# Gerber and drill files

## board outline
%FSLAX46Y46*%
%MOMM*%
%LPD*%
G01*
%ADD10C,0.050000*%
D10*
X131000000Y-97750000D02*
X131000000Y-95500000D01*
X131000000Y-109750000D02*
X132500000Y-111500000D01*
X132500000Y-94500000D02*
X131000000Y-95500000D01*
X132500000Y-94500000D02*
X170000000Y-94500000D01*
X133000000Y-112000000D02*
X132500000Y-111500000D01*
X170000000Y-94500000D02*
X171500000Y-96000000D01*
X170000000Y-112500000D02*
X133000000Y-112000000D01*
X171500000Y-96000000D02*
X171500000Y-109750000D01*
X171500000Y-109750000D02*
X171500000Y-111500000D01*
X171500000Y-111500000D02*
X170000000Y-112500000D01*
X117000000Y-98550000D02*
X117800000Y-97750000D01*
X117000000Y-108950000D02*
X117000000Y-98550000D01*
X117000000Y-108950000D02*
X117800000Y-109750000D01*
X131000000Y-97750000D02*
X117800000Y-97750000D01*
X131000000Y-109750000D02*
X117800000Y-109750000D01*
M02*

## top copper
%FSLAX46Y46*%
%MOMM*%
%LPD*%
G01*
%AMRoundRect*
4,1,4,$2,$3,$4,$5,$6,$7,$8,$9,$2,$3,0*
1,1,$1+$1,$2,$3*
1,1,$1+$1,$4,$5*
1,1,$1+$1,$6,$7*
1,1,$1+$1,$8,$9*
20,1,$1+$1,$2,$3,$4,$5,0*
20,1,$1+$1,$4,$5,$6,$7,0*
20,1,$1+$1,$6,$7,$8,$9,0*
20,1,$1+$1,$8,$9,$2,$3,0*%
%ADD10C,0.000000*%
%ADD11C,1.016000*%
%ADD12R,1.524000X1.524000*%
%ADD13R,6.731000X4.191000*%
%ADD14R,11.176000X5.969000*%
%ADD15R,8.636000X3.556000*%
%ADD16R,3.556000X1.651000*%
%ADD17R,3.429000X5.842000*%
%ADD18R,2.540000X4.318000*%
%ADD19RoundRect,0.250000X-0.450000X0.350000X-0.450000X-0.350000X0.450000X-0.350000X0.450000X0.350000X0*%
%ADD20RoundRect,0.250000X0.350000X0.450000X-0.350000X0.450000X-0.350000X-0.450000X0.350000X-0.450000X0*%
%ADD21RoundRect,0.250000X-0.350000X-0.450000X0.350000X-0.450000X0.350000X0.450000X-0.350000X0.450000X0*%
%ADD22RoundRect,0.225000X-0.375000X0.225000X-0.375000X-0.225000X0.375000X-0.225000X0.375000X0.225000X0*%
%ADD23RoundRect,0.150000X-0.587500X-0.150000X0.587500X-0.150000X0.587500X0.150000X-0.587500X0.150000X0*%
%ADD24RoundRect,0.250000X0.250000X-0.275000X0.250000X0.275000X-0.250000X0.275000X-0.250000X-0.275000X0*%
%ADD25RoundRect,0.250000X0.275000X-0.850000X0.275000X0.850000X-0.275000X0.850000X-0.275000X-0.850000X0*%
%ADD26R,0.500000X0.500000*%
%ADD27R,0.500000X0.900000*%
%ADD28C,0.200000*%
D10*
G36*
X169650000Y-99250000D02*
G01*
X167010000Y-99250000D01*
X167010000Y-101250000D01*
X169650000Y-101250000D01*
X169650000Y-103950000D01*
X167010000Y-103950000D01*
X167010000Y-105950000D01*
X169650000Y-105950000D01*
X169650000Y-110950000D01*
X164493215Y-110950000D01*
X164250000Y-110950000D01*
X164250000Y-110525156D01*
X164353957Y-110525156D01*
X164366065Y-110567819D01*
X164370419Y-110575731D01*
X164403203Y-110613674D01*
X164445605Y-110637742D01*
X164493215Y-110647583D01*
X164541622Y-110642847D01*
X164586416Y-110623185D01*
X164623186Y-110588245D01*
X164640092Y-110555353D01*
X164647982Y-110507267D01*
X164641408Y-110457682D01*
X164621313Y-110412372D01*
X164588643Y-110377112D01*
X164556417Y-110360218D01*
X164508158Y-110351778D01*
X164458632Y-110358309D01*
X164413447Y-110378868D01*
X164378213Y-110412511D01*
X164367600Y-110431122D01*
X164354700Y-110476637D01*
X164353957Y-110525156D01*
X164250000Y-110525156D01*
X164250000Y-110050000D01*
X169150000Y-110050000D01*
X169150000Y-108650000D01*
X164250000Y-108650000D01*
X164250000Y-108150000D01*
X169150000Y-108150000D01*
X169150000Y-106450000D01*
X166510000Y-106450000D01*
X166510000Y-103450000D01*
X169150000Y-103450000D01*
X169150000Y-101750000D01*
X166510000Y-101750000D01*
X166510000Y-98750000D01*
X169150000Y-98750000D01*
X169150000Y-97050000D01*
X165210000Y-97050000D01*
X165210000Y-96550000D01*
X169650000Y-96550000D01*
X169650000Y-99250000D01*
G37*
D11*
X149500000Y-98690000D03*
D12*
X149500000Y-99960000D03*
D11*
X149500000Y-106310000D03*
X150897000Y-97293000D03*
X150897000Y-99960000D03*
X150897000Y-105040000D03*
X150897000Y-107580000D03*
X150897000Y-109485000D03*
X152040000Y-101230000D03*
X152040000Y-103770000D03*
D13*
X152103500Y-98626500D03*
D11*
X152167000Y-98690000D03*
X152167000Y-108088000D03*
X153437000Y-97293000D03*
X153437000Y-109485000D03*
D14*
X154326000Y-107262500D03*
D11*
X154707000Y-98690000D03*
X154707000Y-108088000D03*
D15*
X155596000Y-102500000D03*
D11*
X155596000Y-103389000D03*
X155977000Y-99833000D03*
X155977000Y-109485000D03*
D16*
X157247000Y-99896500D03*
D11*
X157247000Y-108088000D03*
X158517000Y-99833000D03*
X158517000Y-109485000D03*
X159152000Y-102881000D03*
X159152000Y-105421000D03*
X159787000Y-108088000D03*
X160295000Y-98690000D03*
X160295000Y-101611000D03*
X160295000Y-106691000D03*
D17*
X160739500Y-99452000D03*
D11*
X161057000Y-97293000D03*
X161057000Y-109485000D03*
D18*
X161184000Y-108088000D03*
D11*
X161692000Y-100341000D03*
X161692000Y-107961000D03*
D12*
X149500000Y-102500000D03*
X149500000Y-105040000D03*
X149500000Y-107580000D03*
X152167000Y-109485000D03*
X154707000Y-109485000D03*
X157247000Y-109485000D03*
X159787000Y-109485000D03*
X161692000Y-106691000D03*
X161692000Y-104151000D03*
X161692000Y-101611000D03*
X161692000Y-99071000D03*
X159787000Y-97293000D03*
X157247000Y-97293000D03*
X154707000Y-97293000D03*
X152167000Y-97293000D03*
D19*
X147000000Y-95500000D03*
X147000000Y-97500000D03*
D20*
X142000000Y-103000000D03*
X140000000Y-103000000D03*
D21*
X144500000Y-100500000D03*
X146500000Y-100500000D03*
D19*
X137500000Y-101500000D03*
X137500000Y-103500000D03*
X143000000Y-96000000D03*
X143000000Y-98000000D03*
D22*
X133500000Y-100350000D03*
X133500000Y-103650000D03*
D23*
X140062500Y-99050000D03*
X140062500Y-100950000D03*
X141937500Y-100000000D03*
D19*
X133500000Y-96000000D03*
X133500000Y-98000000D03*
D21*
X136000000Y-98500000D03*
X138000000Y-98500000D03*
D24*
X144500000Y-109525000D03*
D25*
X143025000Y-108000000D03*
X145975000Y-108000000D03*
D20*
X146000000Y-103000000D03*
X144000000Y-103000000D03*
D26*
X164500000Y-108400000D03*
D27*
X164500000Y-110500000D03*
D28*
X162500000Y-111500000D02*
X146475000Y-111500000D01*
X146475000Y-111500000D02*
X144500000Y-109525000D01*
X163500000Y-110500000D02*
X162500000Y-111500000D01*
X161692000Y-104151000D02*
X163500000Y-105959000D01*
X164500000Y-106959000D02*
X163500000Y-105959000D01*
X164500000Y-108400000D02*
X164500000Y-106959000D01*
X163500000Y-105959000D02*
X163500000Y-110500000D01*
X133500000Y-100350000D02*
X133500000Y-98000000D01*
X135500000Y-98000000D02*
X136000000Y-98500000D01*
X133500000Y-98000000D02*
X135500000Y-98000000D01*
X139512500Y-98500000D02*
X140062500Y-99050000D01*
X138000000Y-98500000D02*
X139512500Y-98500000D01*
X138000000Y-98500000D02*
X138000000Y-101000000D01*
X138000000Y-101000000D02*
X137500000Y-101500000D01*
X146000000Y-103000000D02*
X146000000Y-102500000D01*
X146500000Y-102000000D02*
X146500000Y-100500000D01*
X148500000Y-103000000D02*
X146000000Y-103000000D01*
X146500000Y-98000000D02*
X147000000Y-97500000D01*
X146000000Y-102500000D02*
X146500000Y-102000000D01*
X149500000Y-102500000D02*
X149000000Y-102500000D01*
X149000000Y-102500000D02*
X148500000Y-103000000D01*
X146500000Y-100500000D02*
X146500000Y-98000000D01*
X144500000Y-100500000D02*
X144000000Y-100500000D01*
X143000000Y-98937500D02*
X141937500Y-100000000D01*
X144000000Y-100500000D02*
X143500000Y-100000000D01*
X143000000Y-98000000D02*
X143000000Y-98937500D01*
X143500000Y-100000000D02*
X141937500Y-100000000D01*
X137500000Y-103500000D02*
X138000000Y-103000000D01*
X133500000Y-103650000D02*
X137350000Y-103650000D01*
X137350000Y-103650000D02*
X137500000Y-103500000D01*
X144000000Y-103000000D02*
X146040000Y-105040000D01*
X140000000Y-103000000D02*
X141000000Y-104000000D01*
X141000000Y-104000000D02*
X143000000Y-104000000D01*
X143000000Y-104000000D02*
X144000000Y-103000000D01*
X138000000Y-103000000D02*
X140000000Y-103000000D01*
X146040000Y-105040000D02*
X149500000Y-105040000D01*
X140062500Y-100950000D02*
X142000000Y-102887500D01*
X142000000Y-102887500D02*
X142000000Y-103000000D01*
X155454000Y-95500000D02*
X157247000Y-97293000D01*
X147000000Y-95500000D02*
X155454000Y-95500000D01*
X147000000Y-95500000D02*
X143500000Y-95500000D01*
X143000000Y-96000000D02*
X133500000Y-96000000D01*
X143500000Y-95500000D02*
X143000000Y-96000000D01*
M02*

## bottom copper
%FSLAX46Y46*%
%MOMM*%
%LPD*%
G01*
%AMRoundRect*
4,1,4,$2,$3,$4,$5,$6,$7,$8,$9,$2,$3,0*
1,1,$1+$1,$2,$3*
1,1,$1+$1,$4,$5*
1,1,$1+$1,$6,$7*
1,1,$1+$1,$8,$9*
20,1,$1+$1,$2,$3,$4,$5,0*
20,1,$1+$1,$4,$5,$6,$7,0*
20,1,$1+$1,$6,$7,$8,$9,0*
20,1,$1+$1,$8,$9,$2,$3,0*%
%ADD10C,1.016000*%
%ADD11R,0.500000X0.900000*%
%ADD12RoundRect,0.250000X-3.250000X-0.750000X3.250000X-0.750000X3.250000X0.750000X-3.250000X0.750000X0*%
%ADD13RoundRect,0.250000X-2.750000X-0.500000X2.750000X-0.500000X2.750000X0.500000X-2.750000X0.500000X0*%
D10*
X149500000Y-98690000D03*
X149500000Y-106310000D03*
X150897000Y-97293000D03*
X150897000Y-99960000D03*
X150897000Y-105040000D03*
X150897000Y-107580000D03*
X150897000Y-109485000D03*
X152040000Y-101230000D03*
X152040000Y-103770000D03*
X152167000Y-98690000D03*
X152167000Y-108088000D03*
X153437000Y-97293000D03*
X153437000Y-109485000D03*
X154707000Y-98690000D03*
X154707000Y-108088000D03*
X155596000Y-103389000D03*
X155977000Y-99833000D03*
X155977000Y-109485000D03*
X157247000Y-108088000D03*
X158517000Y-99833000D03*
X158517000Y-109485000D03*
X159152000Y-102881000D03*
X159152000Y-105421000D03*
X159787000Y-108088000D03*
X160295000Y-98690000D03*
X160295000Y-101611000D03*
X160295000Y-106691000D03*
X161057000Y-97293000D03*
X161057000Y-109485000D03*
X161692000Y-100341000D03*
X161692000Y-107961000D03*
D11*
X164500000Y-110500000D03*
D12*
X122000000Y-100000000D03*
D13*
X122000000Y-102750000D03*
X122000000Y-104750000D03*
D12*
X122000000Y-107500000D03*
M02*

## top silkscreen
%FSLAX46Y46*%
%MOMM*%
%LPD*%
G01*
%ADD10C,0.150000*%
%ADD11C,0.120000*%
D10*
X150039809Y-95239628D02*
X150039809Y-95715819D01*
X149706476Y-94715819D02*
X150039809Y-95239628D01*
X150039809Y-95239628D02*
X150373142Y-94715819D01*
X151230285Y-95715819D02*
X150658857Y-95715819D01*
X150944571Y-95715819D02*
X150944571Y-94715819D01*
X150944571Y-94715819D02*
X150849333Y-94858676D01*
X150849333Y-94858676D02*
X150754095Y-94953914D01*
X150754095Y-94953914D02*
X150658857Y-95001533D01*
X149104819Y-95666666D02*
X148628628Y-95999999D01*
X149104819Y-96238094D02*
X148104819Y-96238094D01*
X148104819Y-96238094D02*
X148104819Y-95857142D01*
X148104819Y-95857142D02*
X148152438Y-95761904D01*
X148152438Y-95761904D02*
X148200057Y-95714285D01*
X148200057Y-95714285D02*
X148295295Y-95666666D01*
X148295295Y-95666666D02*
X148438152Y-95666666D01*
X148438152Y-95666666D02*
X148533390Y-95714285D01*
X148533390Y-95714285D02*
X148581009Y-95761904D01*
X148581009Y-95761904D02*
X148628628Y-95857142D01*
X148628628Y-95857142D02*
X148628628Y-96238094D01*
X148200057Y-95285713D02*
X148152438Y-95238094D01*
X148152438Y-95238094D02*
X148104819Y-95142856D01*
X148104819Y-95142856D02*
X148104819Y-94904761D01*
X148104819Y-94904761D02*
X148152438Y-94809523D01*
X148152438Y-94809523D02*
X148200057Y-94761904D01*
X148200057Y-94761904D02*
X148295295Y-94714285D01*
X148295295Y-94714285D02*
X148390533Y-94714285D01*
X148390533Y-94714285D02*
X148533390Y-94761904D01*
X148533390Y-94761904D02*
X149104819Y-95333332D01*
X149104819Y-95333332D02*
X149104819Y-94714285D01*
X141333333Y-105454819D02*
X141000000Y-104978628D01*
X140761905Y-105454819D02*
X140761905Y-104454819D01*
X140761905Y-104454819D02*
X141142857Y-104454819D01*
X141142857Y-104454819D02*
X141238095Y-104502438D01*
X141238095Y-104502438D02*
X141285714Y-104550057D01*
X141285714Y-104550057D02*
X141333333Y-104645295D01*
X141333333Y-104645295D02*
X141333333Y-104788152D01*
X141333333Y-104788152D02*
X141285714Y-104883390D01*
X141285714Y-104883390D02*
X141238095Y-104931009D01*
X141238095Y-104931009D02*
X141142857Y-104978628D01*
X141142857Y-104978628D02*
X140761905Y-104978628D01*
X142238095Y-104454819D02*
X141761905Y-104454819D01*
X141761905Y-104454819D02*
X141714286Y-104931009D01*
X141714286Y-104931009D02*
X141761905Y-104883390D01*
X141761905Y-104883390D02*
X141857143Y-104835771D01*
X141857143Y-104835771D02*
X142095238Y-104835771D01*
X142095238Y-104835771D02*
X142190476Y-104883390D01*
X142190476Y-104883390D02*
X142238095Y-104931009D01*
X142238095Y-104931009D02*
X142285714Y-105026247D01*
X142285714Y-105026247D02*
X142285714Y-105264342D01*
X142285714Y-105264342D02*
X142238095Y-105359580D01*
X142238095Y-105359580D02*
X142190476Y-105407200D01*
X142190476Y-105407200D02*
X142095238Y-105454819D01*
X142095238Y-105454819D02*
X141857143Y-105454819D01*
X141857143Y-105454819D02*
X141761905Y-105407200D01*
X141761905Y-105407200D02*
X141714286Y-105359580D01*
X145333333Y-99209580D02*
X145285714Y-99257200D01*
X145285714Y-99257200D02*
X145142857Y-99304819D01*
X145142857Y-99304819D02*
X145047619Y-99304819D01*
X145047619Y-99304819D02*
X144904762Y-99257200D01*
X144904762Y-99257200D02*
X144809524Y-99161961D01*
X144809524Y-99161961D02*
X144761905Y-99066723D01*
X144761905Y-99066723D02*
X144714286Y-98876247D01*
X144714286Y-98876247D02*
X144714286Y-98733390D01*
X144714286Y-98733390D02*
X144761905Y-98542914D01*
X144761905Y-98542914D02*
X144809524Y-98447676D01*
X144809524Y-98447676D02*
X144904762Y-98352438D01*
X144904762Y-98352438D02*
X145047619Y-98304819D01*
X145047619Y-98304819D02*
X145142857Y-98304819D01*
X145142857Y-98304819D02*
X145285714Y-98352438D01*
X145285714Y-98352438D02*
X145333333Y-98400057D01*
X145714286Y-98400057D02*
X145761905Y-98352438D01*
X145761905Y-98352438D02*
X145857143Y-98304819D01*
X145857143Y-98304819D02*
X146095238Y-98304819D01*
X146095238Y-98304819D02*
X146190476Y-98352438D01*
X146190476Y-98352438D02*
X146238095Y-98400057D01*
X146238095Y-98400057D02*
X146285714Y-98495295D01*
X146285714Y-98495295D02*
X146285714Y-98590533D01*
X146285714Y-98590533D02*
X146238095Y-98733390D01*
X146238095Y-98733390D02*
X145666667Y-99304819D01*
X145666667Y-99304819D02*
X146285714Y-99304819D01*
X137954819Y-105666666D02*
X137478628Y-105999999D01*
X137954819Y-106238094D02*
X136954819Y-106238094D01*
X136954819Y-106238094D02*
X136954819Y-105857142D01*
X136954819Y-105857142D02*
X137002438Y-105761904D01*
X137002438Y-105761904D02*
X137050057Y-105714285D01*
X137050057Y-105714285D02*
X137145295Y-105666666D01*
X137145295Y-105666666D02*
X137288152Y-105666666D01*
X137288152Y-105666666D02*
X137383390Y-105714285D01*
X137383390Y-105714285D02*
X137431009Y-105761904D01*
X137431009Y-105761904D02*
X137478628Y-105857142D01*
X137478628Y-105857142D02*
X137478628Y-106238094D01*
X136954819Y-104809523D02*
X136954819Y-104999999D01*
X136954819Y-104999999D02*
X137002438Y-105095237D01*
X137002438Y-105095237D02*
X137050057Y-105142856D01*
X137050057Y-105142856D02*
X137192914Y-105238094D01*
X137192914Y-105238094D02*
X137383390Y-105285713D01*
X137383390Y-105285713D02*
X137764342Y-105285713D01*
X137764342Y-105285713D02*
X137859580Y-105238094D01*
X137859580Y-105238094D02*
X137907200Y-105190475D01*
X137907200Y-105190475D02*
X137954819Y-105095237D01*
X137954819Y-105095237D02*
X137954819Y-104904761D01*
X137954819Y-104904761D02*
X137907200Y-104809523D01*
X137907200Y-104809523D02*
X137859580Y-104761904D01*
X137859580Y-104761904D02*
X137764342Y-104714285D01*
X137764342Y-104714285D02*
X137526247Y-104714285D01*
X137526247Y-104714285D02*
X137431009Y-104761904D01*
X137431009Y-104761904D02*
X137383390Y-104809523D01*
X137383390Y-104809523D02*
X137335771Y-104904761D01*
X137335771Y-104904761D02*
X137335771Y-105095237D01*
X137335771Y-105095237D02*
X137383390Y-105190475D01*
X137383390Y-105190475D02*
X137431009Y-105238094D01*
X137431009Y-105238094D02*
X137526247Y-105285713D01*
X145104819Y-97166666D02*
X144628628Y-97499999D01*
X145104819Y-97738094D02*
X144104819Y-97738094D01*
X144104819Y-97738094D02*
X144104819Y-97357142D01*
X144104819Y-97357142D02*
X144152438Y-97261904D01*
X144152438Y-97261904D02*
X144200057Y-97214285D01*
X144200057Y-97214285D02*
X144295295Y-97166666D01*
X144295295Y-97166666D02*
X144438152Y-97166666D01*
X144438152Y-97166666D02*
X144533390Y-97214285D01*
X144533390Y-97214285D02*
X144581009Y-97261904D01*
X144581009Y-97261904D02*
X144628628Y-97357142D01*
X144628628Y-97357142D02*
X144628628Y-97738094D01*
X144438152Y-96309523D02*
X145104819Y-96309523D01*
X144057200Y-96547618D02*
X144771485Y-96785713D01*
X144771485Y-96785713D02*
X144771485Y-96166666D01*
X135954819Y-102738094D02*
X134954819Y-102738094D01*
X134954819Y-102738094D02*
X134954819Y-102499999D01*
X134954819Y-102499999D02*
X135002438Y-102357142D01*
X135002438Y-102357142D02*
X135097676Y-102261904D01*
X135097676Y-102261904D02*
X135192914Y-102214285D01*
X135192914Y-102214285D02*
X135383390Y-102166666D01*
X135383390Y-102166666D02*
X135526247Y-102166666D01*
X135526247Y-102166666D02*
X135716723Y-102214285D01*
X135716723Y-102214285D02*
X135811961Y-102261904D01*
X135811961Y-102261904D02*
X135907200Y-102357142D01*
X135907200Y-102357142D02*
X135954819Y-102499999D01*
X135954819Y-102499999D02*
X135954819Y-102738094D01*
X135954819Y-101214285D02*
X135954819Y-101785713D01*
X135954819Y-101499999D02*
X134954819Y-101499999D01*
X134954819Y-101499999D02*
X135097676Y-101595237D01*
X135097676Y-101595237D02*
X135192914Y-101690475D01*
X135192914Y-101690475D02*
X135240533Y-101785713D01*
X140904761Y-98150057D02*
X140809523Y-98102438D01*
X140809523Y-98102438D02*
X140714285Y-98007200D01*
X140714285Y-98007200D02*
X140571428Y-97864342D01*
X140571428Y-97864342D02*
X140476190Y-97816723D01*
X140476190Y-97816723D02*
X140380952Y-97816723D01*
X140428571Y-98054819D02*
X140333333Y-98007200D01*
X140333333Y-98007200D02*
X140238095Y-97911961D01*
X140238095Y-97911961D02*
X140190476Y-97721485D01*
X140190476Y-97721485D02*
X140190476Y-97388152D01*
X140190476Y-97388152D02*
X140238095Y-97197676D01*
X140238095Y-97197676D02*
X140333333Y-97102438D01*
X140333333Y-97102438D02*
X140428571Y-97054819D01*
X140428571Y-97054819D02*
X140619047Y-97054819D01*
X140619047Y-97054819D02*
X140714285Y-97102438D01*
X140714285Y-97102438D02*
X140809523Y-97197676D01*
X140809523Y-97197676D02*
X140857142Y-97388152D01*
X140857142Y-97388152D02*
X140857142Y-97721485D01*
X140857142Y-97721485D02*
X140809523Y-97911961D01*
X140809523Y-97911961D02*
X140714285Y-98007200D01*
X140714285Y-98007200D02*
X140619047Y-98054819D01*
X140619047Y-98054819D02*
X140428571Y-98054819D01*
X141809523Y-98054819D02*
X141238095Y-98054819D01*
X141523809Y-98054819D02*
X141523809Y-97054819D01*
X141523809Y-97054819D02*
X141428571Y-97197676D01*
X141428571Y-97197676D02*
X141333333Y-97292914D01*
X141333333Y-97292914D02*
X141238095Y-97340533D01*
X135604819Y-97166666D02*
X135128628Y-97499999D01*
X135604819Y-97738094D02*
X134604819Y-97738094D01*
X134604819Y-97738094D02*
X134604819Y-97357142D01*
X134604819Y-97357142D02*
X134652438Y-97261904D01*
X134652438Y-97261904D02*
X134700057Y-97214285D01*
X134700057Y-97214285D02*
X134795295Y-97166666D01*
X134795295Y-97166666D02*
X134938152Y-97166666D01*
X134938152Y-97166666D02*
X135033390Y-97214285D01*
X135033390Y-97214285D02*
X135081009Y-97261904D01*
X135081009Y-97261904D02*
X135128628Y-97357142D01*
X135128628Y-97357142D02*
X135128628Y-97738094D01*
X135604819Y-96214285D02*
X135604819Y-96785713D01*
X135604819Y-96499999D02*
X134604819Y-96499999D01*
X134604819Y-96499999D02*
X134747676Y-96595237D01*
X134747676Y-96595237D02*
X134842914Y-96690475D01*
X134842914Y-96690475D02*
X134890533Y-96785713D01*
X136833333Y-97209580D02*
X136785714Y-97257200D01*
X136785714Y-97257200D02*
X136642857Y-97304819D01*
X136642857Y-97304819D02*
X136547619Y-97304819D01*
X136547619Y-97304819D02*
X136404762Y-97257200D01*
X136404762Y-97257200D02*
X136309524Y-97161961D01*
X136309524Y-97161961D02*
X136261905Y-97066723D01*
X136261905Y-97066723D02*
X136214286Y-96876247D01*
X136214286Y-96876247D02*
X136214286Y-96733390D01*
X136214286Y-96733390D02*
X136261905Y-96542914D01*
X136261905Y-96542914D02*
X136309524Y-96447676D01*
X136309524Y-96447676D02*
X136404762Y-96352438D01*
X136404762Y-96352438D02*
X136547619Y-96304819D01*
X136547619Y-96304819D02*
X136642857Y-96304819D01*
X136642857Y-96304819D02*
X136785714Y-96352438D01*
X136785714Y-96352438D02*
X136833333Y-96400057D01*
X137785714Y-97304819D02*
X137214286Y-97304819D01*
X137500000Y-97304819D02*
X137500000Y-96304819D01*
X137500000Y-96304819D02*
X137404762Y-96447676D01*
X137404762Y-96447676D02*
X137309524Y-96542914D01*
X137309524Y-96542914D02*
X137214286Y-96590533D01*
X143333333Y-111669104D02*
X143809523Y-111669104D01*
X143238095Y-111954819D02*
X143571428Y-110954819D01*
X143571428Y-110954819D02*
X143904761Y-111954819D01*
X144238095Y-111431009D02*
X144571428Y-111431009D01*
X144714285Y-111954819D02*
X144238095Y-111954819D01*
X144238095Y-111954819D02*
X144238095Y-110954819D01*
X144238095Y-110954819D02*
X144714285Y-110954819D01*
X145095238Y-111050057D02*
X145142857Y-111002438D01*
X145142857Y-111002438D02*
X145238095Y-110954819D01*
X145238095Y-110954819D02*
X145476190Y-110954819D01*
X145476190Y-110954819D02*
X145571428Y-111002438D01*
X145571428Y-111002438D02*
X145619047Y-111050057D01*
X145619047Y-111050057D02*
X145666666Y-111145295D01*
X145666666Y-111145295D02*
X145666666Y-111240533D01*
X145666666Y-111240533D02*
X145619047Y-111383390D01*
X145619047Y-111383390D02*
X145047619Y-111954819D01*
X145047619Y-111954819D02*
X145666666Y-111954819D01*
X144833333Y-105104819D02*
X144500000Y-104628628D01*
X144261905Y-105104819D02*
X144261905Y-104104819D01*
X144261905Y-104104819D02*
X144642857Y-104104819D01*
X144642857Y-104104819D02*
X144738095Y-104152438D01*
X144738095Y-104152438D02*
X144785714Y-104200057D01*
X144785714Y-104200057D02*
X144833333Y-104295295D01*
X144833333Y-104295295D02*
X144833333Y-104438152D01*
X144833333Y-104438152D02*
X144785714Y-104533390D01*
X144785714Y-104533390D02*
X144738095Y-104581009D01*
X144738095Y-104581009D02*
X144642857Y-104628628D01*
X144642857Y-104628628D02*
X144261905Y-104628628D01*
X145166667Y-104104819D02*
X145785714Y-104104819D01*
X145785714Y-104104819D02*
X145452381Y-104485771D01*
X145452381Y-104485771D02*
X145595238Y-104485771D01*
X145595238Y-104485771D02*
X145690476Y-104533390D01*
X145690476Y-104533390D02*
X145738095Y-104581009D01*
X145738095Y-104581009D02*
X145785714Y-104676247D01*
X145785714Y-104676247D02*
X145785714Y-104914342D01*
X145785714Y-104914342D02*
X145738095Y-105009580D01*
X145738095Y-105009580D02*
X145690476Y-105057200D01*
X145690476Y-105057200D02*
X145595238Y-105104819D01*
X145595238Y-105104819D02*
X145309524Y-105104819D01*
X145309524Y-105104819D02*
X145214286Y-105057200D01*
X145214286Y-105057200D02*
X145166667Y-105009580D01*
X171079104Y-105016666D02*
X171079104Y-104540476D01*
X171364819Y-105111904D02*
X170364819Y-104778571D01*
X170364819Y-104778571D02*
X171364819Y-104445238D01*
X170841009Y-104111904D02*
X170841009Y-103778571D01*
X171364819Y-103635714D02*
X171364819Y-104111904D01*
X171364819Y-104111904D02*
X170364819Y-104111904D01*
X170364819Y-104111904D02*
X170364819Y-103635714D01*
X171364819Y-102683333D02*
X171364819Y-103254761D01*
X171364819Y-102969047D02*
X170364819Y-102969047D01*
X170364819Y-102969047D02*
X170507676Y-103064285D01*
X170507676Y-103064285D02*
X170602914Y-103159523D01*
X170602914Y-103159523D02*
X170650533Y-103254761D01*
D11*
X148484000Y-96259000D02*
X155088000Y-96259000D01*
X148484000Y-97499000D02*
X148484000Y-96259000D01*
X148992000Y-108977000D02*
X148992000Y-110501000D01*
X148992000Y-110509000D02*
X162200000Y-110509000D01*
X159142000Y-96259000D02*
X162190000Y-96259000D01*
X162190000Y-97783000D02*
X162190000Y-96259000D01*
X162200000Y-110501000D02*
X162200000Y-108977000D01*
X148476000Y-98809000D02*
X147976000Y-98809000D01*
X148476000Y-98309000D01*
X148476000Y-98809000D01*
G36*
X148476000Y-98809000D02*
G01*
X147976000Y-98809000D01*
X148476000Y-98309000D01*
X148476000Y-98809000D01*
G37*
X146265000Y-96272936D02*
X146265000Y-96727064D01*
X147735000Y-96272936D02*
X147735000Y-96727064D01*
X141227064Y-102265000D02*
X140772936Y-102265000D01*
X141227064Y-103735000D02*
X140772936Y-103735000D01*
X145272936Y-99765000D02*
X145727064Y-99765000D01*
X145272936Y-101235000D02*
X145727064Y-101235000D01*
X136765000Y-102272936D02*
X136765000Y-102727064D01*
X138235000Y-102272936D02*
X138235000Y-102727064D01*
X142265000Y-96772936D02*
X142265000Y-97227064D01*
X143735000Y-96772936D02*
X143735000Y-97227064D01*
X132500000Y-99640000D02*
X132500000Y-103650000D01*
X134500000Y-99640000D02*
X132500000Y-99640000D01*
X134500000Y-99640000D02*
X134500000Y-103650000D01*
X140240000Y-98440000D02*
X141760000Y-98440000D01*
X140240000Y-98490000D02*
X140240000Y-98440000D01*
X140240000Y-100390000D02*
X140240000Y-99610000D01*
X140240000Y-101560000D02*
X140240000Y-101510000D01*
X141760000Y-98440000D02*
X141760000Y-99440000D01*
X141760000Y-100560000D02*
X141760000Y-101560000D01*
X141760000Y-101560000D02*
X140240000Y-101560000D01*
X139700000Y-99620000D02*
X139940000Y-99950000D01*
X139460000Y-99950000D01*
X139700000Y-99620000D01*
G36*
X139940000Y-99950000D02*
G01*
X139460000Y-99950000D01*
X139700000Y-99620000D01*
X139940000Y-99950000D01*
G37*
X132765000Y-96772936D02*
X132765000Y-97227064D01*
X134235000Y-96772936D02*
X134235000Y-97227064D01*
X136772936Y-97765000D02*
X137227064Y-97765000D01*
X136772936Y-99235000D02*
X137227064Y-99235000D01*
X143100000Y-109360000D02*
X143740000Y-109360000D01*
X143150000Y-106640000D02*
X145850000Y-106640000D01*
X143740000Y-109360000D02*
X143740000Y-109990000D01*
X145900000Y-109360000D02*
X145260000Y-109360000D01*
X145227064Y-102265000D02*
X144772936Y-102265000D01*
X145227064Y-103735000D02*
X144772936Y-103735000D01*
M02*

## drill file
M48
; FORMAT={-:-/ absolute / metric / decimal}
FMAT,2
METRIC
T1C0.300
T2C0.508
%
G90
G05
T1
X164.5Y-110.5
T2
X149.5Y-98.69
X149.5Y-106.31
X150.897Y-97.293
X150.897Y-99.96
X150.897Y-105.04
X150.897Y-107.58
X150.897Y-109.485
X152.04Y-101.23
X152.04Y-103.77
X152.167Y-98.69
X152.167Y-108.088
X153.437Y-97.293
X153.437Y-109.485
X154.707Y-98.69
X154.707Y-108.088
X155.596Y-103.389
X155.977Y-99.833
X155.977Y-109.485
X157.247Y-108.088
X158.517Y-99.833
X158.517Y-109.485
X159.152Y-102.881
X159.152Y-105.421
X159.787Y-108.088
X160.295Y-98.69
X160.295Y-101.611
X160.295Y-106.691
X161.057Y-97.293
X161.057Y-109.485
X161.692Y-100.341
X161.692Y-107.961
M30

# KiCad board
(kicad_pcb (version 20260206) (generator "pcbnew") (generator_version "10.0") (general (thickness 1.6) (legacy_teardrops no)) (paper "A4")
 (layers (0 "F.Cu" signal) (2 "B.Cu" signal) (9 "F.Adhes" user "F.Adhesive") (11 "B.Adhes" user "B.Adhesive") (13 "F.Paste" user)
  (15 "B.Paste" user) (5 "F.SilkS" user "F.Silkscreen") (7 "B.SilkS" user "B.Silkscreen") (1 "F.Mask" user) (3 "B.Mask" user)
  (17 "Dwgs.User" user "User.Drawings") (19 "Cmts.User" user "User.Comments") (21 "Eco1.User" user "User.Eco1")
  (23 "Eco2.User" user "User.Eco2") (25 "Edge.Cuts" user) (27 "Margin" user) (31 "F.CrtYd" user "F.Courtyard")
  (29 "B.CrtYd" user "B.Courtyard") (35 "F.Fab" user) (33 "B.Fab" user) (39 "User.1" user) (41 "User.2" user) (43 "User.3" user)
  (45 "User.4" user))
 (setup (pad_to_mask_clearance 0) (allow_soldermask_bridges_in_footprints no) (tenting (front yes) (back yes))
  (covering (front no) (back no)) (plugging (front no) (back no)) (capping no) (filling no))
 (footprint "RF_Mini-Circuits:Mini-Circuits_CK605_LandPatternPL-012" (layer "F.Cu") (at 155.596 103.389)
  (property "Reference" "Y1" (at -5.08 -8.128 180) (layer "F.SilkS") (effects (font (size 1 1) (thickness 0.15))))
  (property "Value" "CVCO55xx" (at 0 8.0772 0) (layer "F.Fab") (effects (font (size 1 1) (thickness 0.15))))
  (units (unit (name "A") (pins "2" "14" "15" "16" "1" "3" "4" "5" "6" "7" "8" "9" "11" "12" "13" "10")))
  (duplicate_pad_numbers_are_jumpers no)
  (fp_line (start -7.112 -7.13) (end -0.508 -7.13) (stroke (width 0.12) (type solid)) (layer "F.SilkS"))
  (fp_line (start -7.112 -5.89) (end -7.112 -7.13) (stroke (width 0.12) (type solid)) (layer "F.SilkS"))
  (fp_line (start -6.604 5.588) (end -6.604 7.112) (stroke (width 0.12) (type solid)) (layer "F.SilkS"))
  (fp_line (start -6.604 7.12) (end 6.604 7.12) (stroke (width 0.12) (type solid)) (layer "F.SilkS"))
  (fp_line (start 3.546 -7.13) (end 6.594 -7.13) (stroke (width 0.12) (type solid)) (layer "F.SilkS"))
  (fp_line (start 6.594 -5.606) (end 6.594 -7.13) (stroke (width 0.12) (type solid)) (layer "F.SilkS"))
  (fp_line (start 6.604 7.112) (end 6.604 5.588) (stroke (width 0.12) (type solid)) (layer "F.SilkS"))
  (fp_poly
   (pts (xy -7.12 -4.58) (xy -7.62 -4.58) (xy -7.12 -5.08) (xy -7.12 -4.58)) (stroke (width 0.12) (type solid)) (fill yes) (layer "F.SilkS"))
  (pad "1" thru_hole circle (at -6.096 -4.699) (size 1.016 1.016) (drill 0.508) (layers "*.Cu") (remove_unused_layers no) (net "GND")
   (zone_connect 2))
  (pad "1" smd rect (at -6.096 -3.429 270) (size 1.524 1.524) (layers "F.Cu" "F.Mask" "F.Paste") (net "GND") (zone_connect 2))
  (pad "1" thru_hole circle (at -6.096 2.921) (size 1.016 1.016) (drill 0.508) (layers "*.Cu") (remove_unused_layers no) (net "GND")
   (zone_connect 2))
  (pad "1" thru_hole circle (at -4.699 -6.096) (size 1.016 1.016) (drill 0.508) (layers "*.Cu") (remove_unused_layers no) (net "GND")
   (zone_connect 2))
  (pad "1" thru_hole circle (at -4.699 -3.429) (size 1.016 1.016) (drill 0.508) (layers "*.Cu") (remove_unused_layers no) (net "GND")
   (zone_connect 2))
  (pad "1" thru_hole circle (at -4.699 1.651) (size 1.016 1.016) (drill 0.508) (layers "*.Cu") (remove_unused_layers no) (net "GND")
   (zone_connect 2))
  (pad "1" thru_hole circle (at -4.699 4.191) (size 1.016 1.016) (drill 0.508) (layers "*.Cu") (remove_unused_layers no) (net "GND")
   (zone_connect 2))
  (pad "1" thru_hole circle (at -4.699 6.096) (size 1.016 1.016) (drill 0.508) (layers "*.Cu") (remove_unused_layers no) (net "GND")
   (zone_connect 2))
  (pad "1" thru_hole circle (at -3.556 -2.159) (size 1.016 1.016) (drill 0.508) (layers "*.Cu") (remove_unused_layers no) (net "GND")
   (zone_connect 2))
  (pad "1" thru_hole circle (at -3.556 0.381) (size 1.016 1.016) (drill 0.508) (layers "*.Cu") (remove_unused_layers no) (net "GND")
   (zone_connect 2))
  (pad "1" smd rect (at -3.4925 -4.7625) (size 6.731 4.191) (layers "F.Cu") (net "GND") (zone_connect 2))
  (pad "1" thru_hole circle (at -3.429 -4.699) (size 1.016 1.016) (drill 0.508) (layers "*.Cu") (remove_unused_layers no) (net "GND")
   (zone_connect 2))
  (pad "1" thru_hole circle (at -3.429 4.699) (size 1.016 1.016) (drill 0.508) (layers "*.Cu") (remove_unused_layers no) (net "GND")
   (zone_connect 2))
  (pad "1" thru_hole circle (at -2.159 -6.096) (size 1.016 1.016) (drill 0.508) (layers "*.Cu") (remove_unused_layers no) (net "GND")
   (zone_connect 2))
  (pad "1" thru_hole circle (at -2.159 6.096) (size 1.016 1.016) (drill 0.508) (layers "*.Cu") (remove_unused_layers no) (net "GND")
   (zone_connect 2))
  (pad "1" smd rect (at -1.27 3.8735) (size 11.176 5.969) (layers "F.Cu") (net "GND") (zone_connect 2))
  (pad "1" thru_hole circle (at -0.889 -4.699) (size 1.016 1.016) (drill 0.508) (layers "*.Cu") (remove_unused_layers no) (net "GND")
   (zone_connect 2))
  (pad "1" thru_hole circle (at -0.889 4.699) (size 1.016 1.016) (drill 0.508) (layers "*.Cu") (remove_unused_layers no) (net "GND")
   (zone_connect 2))
  (pad "1" smd rect (at 0 -0.889) (size 8.636 3.556) (layers "F.Cu") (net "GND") (zone_connect 2))
  (pad "1" thru_hole circle (at 0 0) (size 1.016 1.016) (drill 0.508) (layers "*.Cu") (remove_unused_layers no) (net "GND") (zone_connect 2))
  (pad "1" thru_hole circle (at 0.381 -3.556) (size 1.016 1.016) (drill 0.508) (layers "*.Cu") (remove_unused_layers no) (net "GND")
   (zone_connect 2))
  (pad "1" thru_hole circle (at 0.381 6.096) (size 1.016 1.016) (drill 0.508) (layers "*.Cu") (remove_unused_layers no) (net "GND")
   (zone_connect 2))
  (pad "1" smd rect (at 1.651 -3.4925) (size 3.556 1.651) (layers "F.Cu") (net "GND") (zone_connect 2))
  (pad "1" thru_hole circle (at 1.651 4.699) (size 1.016 1.016) (drill 0.508) (layers "*.Cu") (remove_unused_layers no) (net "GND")
   (zone_connect 2))
  (pad "1" thru_hole circle (at 2.921 -3.556) (size 1.016 1.016) (drill 0.508) (layers "*.Cu") (remove_unused_layers no) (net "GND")
   (zone_connect 2))
  (pad "1" thru_hole circle (at 2.921 6.096) (size 1.016 1.016) (drill 0.508) (layers "*.Cu") (remove_unused_layers no) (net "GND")
   (zone_connect 2))
  (pad "1" thru_hole circle (at 3.556 -0.508) (size 1.016 1.016) (drill 0.508) (layers "*.Cu") (remove_unused_layers no) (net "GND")
   (zone_connect 2))
  (pad "1" thru_hole circle (at 3.556 2.032) (size 1.016 1.016) (drill 0.508) (layers "*.Cu") (remove_unused_layers no) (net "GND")
   (zone_connect 2))
  (pad "1" thru_hole circle (at 4.191 4.699) (size 1.016 1.016) (drill 0.508) (layers "*.Cu") (remove_unused_layers no) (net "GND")
   (zone_connect 2))
  (pad "1" thru_hole circle (at 4.699 -4.699) (size 1.016 1.016) (drill 0.508) (layers "*.Cu") (remove_unused_layers no) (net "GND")
   (zone_connect 2))
  (pad "1" thru_hole circle (at 4.699 -1.778) (size 1.016 1.016) (drill 0.508) (layers "*.Cu") (remove_unused_layers no) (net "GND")
   (zone_connect 2))
  (pad "1" thru_hole circle (at 4.699 3.302) (size 1.016 1.016) (drill 0.508) (layers "*.Cu") (remove_unused_layers no) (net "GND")
   (zone_connect 2))
  (pad "1" smd rect (at 5.1435 -3.937) (size 3.429 5.842) (layers "F.Cu") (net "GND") (zone_connect 2))
  (pad "1" thru_hole circle (at 5.461 -6.096) (size 1.016 1.016) (drill 0.508) (layers "*.Cu") (remove_unused_layers no) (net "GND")
   (zone_connect 2))
  (pad "1" thru_hole circle (at 5.461 6.096) (size 1.016 1.016) (drill 0.508) (layers "*.Cu") (remove_unused_layers no) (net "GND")
   (zone_connect 2))
  (pad "1" smd rect (at 5.588 4.699) (size 2.54 4.318) (layers "F.Cu") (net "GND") (zone_connect 2))
  (pad "1" thru_hole circle (at 6.096 -3.048) (size 1.016 1.016) (drill 0.508) (layers "*.Cu") (remove_unused_layers no) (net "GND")
   (zone_connect 2))
  (pad "1" thru_hole circle (at 6.096 4.572) (size 1.016 1.016) (drill 0.508) (layers "*.Cu") (remove_unused_layers no) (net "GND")
   (zone_connect 2))
  (pad "2" smd rect (at -6.096 -0.889 270) (size 1.524 1.524) (layers "F.Cu" "F.Mask" "F.Paste") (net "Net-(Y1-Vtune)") (clearance 1.016))
  (pad "3" smd rect (at -6.096 1.651 270) (size 1.524 1.524) (layers "F.Cu" "F.Mask" "F.Paste") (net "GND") (zone_connect 2))
  (pad "4" smd rect (at -6.096 4.191 270) (size 1.524 1.524) (layers "F.Cu" "F.Mask" "F.Paste") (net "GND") (zone_connect 2))
  (pad "5" smd rect (at -3.429 6.096 270) (size 1.524 1.524) (layers "F.Cu" "F.Mask" "F.Paste") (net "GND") (zone_connect 2))
  (pad "6" smd rect (at -0.889 6.096 270) (size 1.524 1.524) (layers "F.Cu" "F.Mask" "F.Paste") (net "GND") (zone_connect 2))
  (pad "7" smd rect (at 1.651 6.096 270) (size 1.524 1.524) (layers "F.Cu" "F.Mask" "F.Paste") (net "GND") (zone_connect 2))
  (pad "8" smd rect (at 4.191 6.096 270) (size 1.524 1.524) (layers "F.Cu" "F.Mask" "F.Paste") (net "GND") (zone_connect 2))
  (pad "9" smd rect (at 6.096 3.302 270) (size 1.524 1.524) (layers "F.Cu" "F.Mask" "F.Paste") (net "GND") (zone_connect 2))
  (pad "10" smd rect (at 6.096 0.762 270) (size 1.524 1.524) (layers "F.Cu" "F.Mask" "F.Paste") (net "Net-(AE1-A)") (clearance 1.016))
  (pad "11" smd rect (at 6.096 -1.778 270) (size 1.524 1.524) (layers "F.Cu" "F.Mask" "F.Paste") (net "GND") (zone_connect 2))
  (pad "12" smd rect (at 6.096 -4.318 270) (size 1.524 1.524) (layers "F.Cu" "F.Mask" "F.Paste") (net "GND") (zone_connect 2))
  (pad "13" smd rect (at 4.191 -6.096 270) (size 1.524 1.524) (layers "F.Cu" "F.Mask" "F.Paste") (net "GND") (zone_connect 2))
  (pad "14" smd rect (at 1.651 -6.096 270) (size 1.524 1.524) (layers "F.Cu" "F.Mask" "F.Paste") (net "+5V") (clearance 1.016))
  (pad "15" smd rect (at -0.889 -6.096 270) (size 1.524 1.524) (layers "F.Cu" "F.Mask" "F.Paste") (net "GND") (zone_connect 2))
  (pad "16" smd rect (at -3.429 -6.096 270) (size 1.524 1.524) (layers "F.Cu" "F.Mask" "F.Paste") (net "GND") (zone_connect 2)))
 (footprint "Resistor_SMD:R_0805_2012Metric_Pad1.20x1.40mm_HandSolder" (layer "F.Cu") (at 147 96.5 -90)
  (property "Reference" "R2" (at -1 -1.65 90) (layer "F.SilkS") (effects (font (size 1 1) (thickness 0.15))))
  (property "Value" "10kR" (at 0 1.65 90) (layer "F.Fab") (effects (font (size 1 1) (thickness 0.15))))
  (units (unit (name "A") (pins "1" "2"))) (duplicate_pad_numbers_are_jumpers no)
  (fp_line (start -0.227064 0.735) (end 0.227064 0.735) (stroke (width 0.12) (type solid)) (layer "F.SilkS"))
  (fp_line (start -0.227064 -0.735) (end 0.227064 -0.735) (stroke (width 0.12) (type solid)) (layer "F.SilkS"))
  (pad "1" smd roundrect (at -1 0 270) (size 1.2 1.4) (layers "F.Cu" "F.Mask" "F.Paste") (roundrect_rratio 0.208333) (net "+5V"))
  (pad "2" smd roundrect (at 1 0 270) (size 1.2 1.4) (layers "F.Cu" "F.Mask" "F.Paste") (roundrect_rratio 0.208333) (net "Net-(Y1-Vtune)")))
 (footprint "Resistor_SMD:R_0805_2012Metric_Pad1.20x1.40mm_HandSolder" (layer "F.Cu") (at 141 103 180)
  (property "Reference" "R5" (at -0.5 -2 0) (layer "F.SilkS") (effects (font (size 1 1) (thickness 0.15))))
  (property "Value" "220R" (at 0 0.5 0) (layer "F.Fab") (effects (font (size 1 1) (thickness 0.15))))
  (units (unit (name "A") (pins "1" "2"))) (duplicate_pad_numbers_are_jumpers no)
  (fp_line (start -0.227064 0.735) (end 0.227064 0.735) (stroke (width 0.12) (type solid)) (layer "F.SilkS"))
  (fp_line (start -0.227064 -0.735) (end 0.227064 -0.735) (stroke (width 0.12) (type solid)) (layer "F.SilkS"))
  (pad "1" smd roundrect (at -1 0 180) (size 1.2 1.4) (layers "F.Cu" "F.Mask" "F.Paste") (roundrect_rratio 0.208333) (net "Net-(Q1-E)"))
  (pad "2" smd roundrect (at 1 0 180) (size 1.2 1.4) (layers "F.Cu" "F.Mask" "F.Paste") (roundrect_rratio 0.208333) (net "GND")))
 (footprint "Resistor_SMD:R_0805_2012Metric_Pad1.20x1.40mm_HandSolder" (layer "F.Cu") (at 145.5 100.5)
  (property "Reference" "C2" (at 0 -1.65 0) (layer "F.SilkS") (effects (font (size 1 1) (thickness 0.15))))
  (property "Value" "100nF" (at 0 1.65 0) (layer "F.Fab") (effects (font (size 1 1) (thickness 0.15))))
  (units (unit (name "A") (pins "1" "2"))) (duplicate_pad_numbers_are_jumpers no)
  (fp_line (start -0.227064 -0.735) (end 0.227064 -0.735) (stroke (width 0.12) (type solid)) (layer "F.SilkS"))
  (fp_line (start -0.227064 0.735) (end 0.227064 0.735) (stroke (width 0.12) (type solid)) (layer "F.SilkS"))
  (pad "1" smd roundrect (at -1 0) (size 1.2 1.4) (layers "F.Cu" "F.Mask" "F.Paste") (roundrect_rratio 0.208333) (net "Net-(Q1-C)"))
  (pad "2" smd roundrect (at 1 0) (size 1.2 1.4) (layers "F.Cu" "F.Mask" "F.Paste") (roundrect_rratio 0.208333) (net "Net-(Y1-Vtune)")))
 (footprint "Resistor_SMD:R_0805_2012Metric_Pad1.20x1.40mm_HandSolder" (layer "F.Cu") (at 137.5 102.5 -90)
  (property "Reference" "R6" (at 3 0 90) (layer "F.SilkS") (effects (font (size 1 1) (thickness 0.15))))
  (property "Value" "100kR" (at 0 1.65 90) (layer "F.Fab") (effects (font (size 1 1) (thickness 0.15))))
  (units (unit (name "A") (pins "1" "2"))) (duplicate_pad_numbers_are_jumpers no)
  (fp_line (start -0.227064 0.735) (end 0.227064 0.735) (stroke (width 0.12) (type solid)) (layer "F.SilkS"))
  (fp_line (start -0.227064 -0.735) (end 0.227064 -0.735) (stroke (width 0.12) (type solid)) (layer "F.SilkS"))
  (pad "1" smd roundrect (at -1 0 270) (size 1.2 1.4) (layers "F.Cu" "F.Mask" "F.Paste") (roundrect_rratio 0.208333) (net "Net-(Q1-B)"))
  (pad "2" smd roundrect (at 1 0 270) (size 1.2 1.4) (layers "F.Cu" "F.Mask" "F.Paste") (roundrect_rratio 0.208333) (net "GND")))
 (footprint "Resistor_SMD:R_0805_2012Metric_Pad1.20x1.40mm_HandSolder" (layer "F.Cu") (at 143 97 -90)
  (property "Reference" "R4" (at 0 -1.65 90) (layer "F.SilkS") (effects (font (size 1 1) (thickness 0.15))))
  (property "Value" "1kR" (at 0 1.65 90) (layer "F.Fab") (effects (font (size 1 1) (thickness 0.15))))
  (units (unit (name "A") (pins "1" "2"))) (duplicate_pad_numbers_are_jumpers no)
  (fp_line (start -0.227064 0.735) (end 0.227064 0.735) (stroke (width 0.12) (type solid)) (layer "F.SilkS"))
  (fp_line (start -0.227064 -0.735) (end 0.227064 -0.735) (stroke (width 0.12) (type solid)) (layer "F.SilkS"))
  (pad "1" smd roundrect (at -1 0 270) (size 1.2 1.4) (layers "F.Cu" "F.Mask" "F.Paste") (roundrect_rratio 0.208333) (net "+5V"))
  (pad "2" smd roundrect (at 1 0 270) (size 1.2 1.4) (layers "F.Cu" "F.Mask" "F.Paste") (roundrect_rratio 0.208333) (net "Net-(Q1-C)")))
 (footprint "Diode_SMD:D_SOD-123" (layer "F.Cu") (at 133.5 102 -90)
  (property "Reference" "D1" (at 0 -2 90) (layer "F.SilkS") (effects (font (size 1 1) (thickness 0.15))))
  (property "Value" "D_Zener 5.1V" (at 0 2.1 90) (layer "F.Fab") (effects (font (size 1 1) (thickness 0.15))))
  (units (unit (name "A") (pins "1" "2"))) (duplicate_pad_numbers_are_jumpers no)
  (fp_line (start -2.36 1) (end 1.65 1) (stroke (width 0.12) (type solid)) (layer "F.SilkS"))
  (fp_line (start -2.36 -1) (end -2.36 1) (stroke (width 0.12) (type solid)) (layer "F.SilkS"))
  (fp_line (start -2.36 -1) (end 1.65 -1) (stroke (width 0.12) (type solid)) (layer "F.SilkS"))
  (pad "1" smd roundrect (at -1.65 0 270) (size 0.9 1.2) (layers "F.Cu" "F.Mask" "F.Paste") (roundrect_rratio 0.25) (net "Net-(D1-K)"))
  (pad "2" smd roundrect (at 1.65 0 270) (size 0.9 1.2) (layers "F.Cu" "F.Mask" "F.Paste") (roundrect_rratio 0.25) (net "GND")))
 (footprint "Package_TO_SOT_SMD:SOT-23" (layer "F.Cu") (at 141 100)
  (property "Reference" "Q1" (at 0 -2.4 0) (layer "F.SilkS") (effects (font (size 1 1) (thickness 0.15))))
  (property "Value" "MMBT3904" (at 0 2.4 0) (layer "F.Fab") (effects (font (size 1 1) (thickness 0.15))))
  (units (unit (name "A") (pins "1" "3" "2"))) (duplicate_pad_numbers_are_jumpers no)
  (fp_line (start -0.76 -1.56) (end 0.76 -1.56) (stroke (width 0.12) (type solid)) (layer "F.SilkS"))
  (fp_line (start -0.76 -1.51) (end -0.76 -1.56) (stroke (width 0.12) (type solid)) (layer "F.SilkS"))
  (fp_line (start -0.76 0.39) (end -0.76 -0.39) (stroke (width 0.12) (type solid)) (layer "F.SilkS"))
  (fp_line (start -0.76 1.56) (end -0.76 1.51) (stroke (width 0.12) (type solid)) (layer "F.SilkS"))
  (fp_line (start 0.76 -1.56) (end 0.76 -0.56) (stroke (width 0.12) (type solid)) (layer "F.SilkS"))
  (fp_line (start 0.76 0.56) (end 0.76 1.56) (stroke (width 0.12) (type solid)) (layer "F.SilkS"))
  (fp_line (start 0.76 1.56) (end -0.76 1.56) (stroke (width 0.12) (type solid)) (layer "F.SilkS"))
  (fp_poly (pts (xy -1.3 -0.38) (xy -1.06 -0.05) (xy -1.54 -0.05)) (stroke (width 0.12) (type solid)) (fill yes) (layer "F.SilkS"))
  (pad "1" smd roundrect (at -0.9375 -0.95) (size 1.475 0.6) (layers "F.Cu" "F.Mask" "F.Paste") (roundrect_rratio 0.25) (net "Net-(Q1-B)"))
  (pad "2" smd roundrect (at -0.9375 0.95) (size 1.475 0.6) (layers "F.Cu" "F.Mask" "F.Paste") (roundrect_rratio 0.25) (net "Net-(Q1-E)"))
  (pad "3" smd roundrect (at 0.9375 0) (size 1.475 0.6) (layers "F.Cu" "F.Mask" "F.Paste") (roundrect_rratio 0.25) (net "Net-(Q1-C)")))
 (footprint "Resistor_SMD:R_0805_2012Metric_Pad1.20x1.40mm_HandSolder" (layer "F.Cu") (at 133.5 97 -90)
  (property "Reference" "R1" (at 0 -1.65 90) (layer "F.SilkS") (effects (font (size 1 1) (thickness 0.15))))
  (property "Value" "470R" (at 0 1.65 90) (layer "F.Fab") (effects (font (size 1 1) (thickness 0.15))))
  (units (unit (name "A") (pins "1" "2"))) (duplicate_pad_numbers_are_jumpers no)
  (fp_line (start -0.227064 0.735) (end 0.227064 0.735) (stroke (width 0.12) (type solid)) (layer "F.SilkS"))
  (fp_line (start -0.227064 -0.735) (end 0.227064 -0.735) (stroke (width 0.12) (type solid)) (layer "F.SilkS"))
  (pad "1" smd roundrect (at -1 0 270) (size 1.2 1.4) (layers "F.Cu" "F.Mask" "F.Paste") (roundrect_rratio 0.208333) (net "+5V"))
  (pad "2" smd roundrect (at 1 0 270) (size 1.2 1.4) (layers "F.Cu" "F.Mask" "F.Paste") (roundrect_rratio 0.208333) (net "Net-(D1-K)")))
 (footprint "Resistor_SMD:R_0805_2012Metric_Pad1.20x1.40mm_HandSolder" (layer "F.Cu") (at 137 98.5)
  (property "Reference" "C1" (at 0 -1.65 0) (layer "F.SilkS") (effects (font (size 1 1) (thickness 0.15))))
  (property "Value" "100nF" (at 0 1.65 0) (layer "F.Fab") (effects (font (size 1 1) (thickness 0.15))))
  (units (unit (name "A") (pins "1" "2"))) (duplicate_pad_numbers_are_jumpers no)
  (fp_line (start -0.227064 -0.735) (end 0.227064 -0.735) (stroke (width 0.12) (type solid)) (layer "F.SilkS"))
  (fp_line (start -0.227064 0.735) (end 0.227064 0.735) (stroke (width 0.12) (type solid)) (layer "F.SilkS"))
  (pad "1" smd roundrect (at -1 0) (size 1.2 1.4) (layers "F.Cu" "F.Mask" "F.Paste") (roundrect_rratio 0.208333) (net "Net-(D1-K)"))
  (pad "2" smd roundrect (at 1 0) (size 1.2 1.4) (layers "F.Cu" "F.Mask" "F.Paste") (roundrect_rratio 0.208333) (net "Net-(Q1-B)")))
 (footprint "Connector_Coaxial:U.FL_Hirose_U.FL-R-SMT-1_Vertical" (layer "F.Cu") (at 144.5 108 90)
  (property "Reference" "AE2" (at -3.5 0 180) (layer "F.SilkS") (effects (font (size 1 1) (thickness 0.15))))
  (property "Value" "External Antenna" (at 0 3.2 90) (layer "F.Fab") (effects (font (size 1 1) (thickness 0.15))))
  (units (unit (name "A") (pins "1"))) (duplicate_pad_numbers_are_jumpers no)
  (fp_line (start -1.36 -1.4) (end -1.36 -0.76) (stroke (width 0.12) (type solid)) (layer "F.SilkS"))
  (fp_line (start 1.36 -1.35) (end 1.36 1.35) (stroke (width 0.12) (type solid)) (layer "F.SilkS"))
  (fp_line (start -1.36 -0.76) (end -1.99 -0.76) (stroke (width 0.12) (type solid)) (layer "F.SilkS"))
  (fp_line (start -1.36 1.4) (end -1.36 0.76) (stroke (width 0.12) (type solid)) (layer "F.SilkS"))
  (pad "1" smd roundrect (at -1.525 0 90) (size 1.05 1) (layers "F.Cu" "F.Mask" "F.Paste") (roundrect_rratio 0.25) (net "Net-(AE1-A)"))
  (pad "2" smd roundrect (at 0 -1.475 90) (size 2.2 1.05) (layers "F.Cu" "F.Mask" "F.Paste") (roundrect_rratio 0.2380952381))
  (pad "2" smd roundrect (at 0 1.475 90) (size 2.2 1.05) (layers "F.Cu" "F.Mask" "F.Paste") (roundrect_rratio 0.2380952381))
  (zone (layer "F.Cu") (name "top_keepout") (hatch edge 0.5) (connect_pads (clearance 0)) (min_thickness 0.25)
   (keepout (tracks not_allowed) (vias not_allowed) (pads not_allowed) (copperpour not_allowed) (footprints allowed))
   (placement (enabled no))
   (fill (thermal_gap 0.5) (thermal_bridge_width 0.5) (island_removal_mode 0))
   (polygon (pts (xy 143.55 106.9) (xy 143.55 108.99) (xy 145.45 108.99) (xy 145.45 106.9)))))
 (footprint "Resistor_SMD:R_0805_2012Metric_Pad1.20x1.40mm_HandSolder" (layer "F.Cu") (at 145 103 180)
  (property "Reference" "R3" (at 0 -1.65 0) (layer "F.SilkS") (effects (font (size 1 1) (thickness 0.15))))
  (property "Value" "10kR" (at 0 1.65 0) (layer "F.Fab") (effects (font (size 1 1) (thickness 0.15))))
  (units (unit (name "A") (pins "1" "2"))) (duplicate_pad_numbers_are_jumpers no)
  (fp_line (start -0.227064 0.735) (end 0.227064 0.735) (stroke (width 0.12) (type solid)) (layer "F.SilkS"))
  (fp_line (start -0.227064 -0.735) (end 0.227064 -0.735) (stroke (width 0.12) (type solid)) (layer "F.SilkS"))
  (pad "1" smd roundrect (at -1 0 180) (size 1.2 1.4) (layers "F.Cu" "F.Mask" "F.Paste") (roundrect_rratio 0.208333) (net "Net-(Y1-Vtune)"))
  (pad "2" smd roundrect (at 1 0 180) (size 1.2 1.4) (layers "F.Cu" "F.Mask" "F.Paste") (roundrect_rratio 0.208333) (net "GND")))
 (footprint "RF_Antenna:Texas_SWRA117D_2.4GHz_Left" (layer "F.Cu") (at 164.5 108.4 -90)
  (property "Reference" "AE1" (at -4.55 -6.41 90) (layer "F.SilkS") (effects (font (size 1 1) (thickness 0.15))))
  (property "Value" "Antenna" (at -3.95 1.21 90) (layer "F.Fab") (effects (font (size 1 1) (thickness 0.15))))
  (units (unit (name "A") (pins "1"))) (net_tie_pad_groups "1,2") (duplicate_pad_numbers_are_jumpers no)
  (fp_poly
   (pts (xy -2.45 -2.51) (xy -4.45 -2.51) (xy -4.45 -5.15) (xy -7.15 -5.15) (xy -7.15 -2.51) (xy -9.15 -2.51) (xy -9.15 -5.15)
    (xy -11.85 -5.15) (xy -11.85 -0.71) (xy -11.35 -0.71) (xy -11.35 -4.65) (xy -9.65 -4.65) (xy -9.65 -2.01) (xy -6.65 -2.01)
    (xy -6.65 -4.65) (xy -4.95 -4.65) (xy -4.95 -2.01) (xy -1.95 -2.01) (xy -1.95 -4.65) (xy -0.25 -4.65) (xy -0.25 0.25) (xy 0.25 0.25)
    (xy 0.25 -4.65) (xy 1.65 -4.65) (xy 1.65 0.25) (xy 2.55 0.25) (xy 2.55 0.006785) (xy 2.247583 0.006785) (xy 2.237742 0.054395)
    (xy 2.213674 0.096797) (xy 2.175731 0.129581) (xy 2.167819 0.133935) (xy 2.125156 0.146043) (xy 2.076637 0.1453) (xy 2.031122 0.1324)
    (xy 2.012511 0.121787) (xy 1.978868 0.086553) (xy 1.958309 0.041368) (xy 1.951778 -0.008158) (xy 1.960218 -0.056417)
    (xy 1.977112 -0.088643) (xy 2.012372 -0.121313) (xy 2.057682 -0.141408) (xy 2.107267 -0.147982) (xy 2.155353 -0.140092)
    (xy 2.188245 -0.123186) (xy 2.223185 -0.086416) (xy 2.242847 -0.041622) (xy 2.247583 0.006785) (xy 2.55 0.006785) (xy 2.55 -5.15)
    (xy -2.45 -5.15) (xy -2.45 -2.51))
   (stroke (width 0) (type solid)) (fill yes) (layer "F.Cu"))
  (pad "1" connect rect (at 0 0 270) (size 0.5 0.5) (layers "F.Cu") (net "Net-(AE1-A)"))
  (pad "2" thru_hole rect (at 2.1 0 270) (size 0.9 0.5) (drill 0.3) (layers "*.Cu") (remove_unused_layers no) (zone_connect 2)))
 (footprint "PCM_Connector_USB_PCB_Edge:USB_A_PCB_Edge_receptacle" (layer "B.Cu") (at 122 103.75)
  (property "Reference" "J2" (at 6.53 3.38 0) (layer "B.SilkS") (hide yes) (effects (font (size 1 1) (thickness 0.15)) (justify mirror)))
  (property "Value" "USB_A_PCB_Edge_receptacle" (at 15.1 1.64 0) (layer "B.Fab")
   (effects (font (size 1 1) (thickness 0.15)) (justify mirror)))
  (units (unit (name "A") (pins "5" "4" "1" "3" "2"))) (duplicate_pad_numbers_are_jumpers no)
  (fp_line (start -5 -5.2) (end -4.2 -6) (stroke (width 0.05) (type default)) (layer "Edge.Cuts"))
  (fp_line (start -5 5.2) (end -5 -5.2) (stroke (width 0.05) (type default)) (layer "Edge.Cuts"))
  (fp_line (start -5 5.2) (end -4.2 6) (stroke (width 0.05) (type default)) (layer "Edge.Cuts"))
  (fp_line (start 9 -6) (end -4.2 -6) (stroke (width 0.05) (type default)) (layer "Edge.Cuts"))
  (fp_line (start 9 6) (end -4.2 6) (stroke (width 0.05) (type default)) (layer "Edge.Cuts"))
  (pad "1" smd roundrect (at 0 -3.75) (size 7 2) (layers "B.Cu" "B.Mask") (roundrect_rratio 0.125) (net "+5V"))
  (pad "2" smd roundrect (at 0 -1) (size 6 1.5) (layers "B.Cu" "B.Mask") (roundrect_rratio 0.1666666667) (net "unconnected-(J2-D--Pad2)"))
  (pad "3" smd roundrect (at 0 1) (size 6 1.5) (layers "B.Cu" "B.Mask") (roundrect_rratio 0.1666666667) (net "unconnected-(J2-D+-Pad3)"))
  (pad "4" smd roundrect (at 0 3.75) (size 7 2) (layers "B.Cu" "B.Mask") (roundrect_rratio 0.125) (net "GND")))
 (gr_line (start 131 97.75) (end 131 95.5) (stroke (width 0.05) (type default)) (layer "Edge.Cuts"))
 (gr_line (start 131 109.75) (end 132.5 111.5) (stroke (width 0.05) (type default)) (layer "Edge.Cuts"))
 (gr_line (start 132.5 94.5) (end 131 95.5) (stroke (width 0.05) (type default)) (layer "Edge.Cuts"))
 (gr_line (start 132.5 94.5) (end 170 94.5) (stroke (width 0.05) (type default)) (layer "Edge.Cuts"))
 (gr_line (start 133 112) (end 132.5 111.5) (stroke (width 0.05) (type default)) (layer "Edge.Cuts"))
 (gr_line (start 170 94.5) (end 171.5 96) (stroke (width 0.05) (type default)) (layer "Edge.Cuts"))
 (gr_line (start 170 112.5) (end 133 112) (stroke (width 0.05) (type default)) (layer "Edge.Cuts"))
 (gr_line (start 171.5 96) (end 171.5 109.75) (stroke (width 0.05) (type default)) (layer "Edge.Cuts"))
 (gr_line (start 171.5 109.75) (end 171.5 111.5) (stroke (width 0.05) (type default)) (layer "Edge.Cuts"))
 (gr_line (start 171.5 111.5) (end 170 112.5) (stroke (width 0.05) (type default)) (layer "Edge.Cuts"))
 (segment (start 162.5 111.5) (end 146.475 111.5) (width 0.2) (layer "F.Cu") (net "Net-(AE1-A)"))
 (segment (start 146.475 111.5) (end 144.5 109.525) (width 0.2) (layer "F.Cu") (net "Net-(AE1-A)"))
 (segment (start 163.5 110.5) (end 162.5 111.5) (width 0.2) (layer "F.Cu") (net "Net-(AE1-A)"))
 (segment (start 161.692 104.151) (end 163.5 105.959) (width 0.2) (layer "F.Cu") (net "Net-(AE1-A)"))
 (segment (start 164.5 106.959) (end 163.5 105.959) (width 0.2) (layer "F.Cu") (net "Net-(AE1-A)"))
 (segment (start 164.5 108.4) (end 164.5 106.959) (width 0.2) (layer "F.Cu") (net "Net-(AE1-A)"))
 (segment (start 163.5 105.959) (end 163.5 110.5) (width 0.2) (layer "F.Cu") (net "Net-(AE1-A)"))
 (segment (start 133.5 100.35) (end 133.5 98) (width 0.2) (layer "F.Cu") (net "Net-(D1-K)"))
 (segment (start 135.5 98) (end 136 98.5) (width 0.2) (layer "F.Cu") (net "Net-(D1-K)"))
 (segment (start 133.5 98) (end 135.5 98) (width 0.2) (layer "F.Cu") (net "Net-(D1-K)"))
 (segment (start 139.5125 98.5) (end 140.0625 99.05) (width 0.2) (layer "F.Cu") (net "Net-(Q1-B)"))
 (segment (start 138 98.5) (end 139.5125 98.5) (width 0.2) (layer "F.Cu") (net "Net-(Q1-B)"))
 (segment (start 138 98.5) (end 138 101) (width 0.2) (layer "F.Cu") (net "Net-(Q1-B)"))
 (segment (start 138 101) (end 137.5 101.5) (width 0.2) (layer "F.Cu") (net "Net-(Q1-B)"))
 (segment (start 146 103) (end 146 102.5) (width 0.2) (layer "F.Cu") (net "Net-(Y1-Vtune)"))
 (segment (start 146.5 102) (end 146.5 100.5) (width 0.2) (layer "F.Cu") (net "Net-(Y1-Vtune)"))
 (segment (start 148.5 103) (end 146 103) (width 0.2) (layer "F.Cu") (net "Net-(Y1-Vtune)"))
 (segment (start 146.5 98) (end 147 97.5) (width 0.2) (layer "F.Cu") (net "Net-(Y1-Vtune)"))
 (segment (start 146 102.5) (end 146.5 102) (width 0.2) (layer "F.Cu") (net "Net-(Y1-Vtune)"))
 (segment (start 149.5 102.5) (end 149 102.5) (width 0.2) (layer "F.Cu") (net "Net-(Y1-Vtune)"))
 (segment (start 149 102.5) (end 148.5 103) (width 0.2) (layer "F.Cu") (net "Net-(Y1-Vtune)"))
 (segment (start 146.5 100.5) (end 146.5 98) (width 0.2) (layer "F.Cu") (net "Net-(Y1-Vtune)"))
 (segment (start 144.5 100.5) (end 144 100.5) (width 0.2) (layer "F.Cu") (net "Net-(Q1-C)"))
 (segment (start 143 98.9375) (end 141.9375 100) (width 0.2) (layer "F.Cu") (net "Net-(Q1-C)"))
 (segment (start 144 100.5) (end 143.5 100) (width 0.2) (layer "F.Cu") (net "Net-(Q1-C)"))
 (segment (start 143 98) (end 143 98.9375) (width 0.2) (layer "F.Cu") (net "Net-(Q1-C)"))
 (segment (start 143.5 100) (end 141.9375 100) (width 0.2) (layer "F.Cu") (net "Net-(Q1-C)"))
 (segment (start 137.5 103.5) (end 138 103) (width 0.2) (layer "F.Cu") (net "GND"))
 (segment (start 133.5 103.65) (end 137.35 103.65) (width 0.2) (layer "F.Cu") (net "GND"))
 (segment (start 137.35 103.65) (end 137.5 103.5) (width 0.2) (layer "F.Cu") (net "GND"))
 (segment (start 144 103) (end 146.04 105.04) (width 0.2) (layer "F.Cu") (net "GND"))
 (segment (start 140 103) (end 141 104) (width 0.2) (layer "F.Cu") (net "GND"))
 (segment (start 141 104) (end 143 104) (width 0.2) (layer "F.Cu") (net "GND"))
 (segment (start 143 104) (end 144 103) (width 0.2) (layer "F.Cu") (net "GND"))
 (segment (start 138 103) (end 140 103) (width 0.2) (layer "F.Cu") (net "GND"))
 (segment (start 146.04 105.04) (end 149.5 105.04) (width 0.2) (layer "F.Cu") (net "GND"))
 (segment (start 140.0625 100.95) (end 142 102.8875) (width 0.2) (layer "F.Cu") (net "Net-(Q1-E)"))
 (segment (start 142 102.8875) (end 142 103) (width 0.2) (layer "F.Cu") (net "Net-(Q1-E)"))
 (segment (start 155.454 95.5) (end 157.247 97.293) (width 0.2) (layer "F.Cu") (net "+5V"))
 (segment (start 147 95.5) (end 155.454 95.5) (width 0.2) (layer "F.Cu") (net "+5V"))
 (segment (start 147 95.5) (end 143.5 95.5) (width 0.2) (layer "F.Cu") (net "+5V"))
 (segment (start 143 96) (end 133.5 96) (width 0.2) (layer "F.Cu") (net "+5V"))
 (segment (start 143.5 95.5) (end 143 96) (width 0.2) (layer "F.Cu") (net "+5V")))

